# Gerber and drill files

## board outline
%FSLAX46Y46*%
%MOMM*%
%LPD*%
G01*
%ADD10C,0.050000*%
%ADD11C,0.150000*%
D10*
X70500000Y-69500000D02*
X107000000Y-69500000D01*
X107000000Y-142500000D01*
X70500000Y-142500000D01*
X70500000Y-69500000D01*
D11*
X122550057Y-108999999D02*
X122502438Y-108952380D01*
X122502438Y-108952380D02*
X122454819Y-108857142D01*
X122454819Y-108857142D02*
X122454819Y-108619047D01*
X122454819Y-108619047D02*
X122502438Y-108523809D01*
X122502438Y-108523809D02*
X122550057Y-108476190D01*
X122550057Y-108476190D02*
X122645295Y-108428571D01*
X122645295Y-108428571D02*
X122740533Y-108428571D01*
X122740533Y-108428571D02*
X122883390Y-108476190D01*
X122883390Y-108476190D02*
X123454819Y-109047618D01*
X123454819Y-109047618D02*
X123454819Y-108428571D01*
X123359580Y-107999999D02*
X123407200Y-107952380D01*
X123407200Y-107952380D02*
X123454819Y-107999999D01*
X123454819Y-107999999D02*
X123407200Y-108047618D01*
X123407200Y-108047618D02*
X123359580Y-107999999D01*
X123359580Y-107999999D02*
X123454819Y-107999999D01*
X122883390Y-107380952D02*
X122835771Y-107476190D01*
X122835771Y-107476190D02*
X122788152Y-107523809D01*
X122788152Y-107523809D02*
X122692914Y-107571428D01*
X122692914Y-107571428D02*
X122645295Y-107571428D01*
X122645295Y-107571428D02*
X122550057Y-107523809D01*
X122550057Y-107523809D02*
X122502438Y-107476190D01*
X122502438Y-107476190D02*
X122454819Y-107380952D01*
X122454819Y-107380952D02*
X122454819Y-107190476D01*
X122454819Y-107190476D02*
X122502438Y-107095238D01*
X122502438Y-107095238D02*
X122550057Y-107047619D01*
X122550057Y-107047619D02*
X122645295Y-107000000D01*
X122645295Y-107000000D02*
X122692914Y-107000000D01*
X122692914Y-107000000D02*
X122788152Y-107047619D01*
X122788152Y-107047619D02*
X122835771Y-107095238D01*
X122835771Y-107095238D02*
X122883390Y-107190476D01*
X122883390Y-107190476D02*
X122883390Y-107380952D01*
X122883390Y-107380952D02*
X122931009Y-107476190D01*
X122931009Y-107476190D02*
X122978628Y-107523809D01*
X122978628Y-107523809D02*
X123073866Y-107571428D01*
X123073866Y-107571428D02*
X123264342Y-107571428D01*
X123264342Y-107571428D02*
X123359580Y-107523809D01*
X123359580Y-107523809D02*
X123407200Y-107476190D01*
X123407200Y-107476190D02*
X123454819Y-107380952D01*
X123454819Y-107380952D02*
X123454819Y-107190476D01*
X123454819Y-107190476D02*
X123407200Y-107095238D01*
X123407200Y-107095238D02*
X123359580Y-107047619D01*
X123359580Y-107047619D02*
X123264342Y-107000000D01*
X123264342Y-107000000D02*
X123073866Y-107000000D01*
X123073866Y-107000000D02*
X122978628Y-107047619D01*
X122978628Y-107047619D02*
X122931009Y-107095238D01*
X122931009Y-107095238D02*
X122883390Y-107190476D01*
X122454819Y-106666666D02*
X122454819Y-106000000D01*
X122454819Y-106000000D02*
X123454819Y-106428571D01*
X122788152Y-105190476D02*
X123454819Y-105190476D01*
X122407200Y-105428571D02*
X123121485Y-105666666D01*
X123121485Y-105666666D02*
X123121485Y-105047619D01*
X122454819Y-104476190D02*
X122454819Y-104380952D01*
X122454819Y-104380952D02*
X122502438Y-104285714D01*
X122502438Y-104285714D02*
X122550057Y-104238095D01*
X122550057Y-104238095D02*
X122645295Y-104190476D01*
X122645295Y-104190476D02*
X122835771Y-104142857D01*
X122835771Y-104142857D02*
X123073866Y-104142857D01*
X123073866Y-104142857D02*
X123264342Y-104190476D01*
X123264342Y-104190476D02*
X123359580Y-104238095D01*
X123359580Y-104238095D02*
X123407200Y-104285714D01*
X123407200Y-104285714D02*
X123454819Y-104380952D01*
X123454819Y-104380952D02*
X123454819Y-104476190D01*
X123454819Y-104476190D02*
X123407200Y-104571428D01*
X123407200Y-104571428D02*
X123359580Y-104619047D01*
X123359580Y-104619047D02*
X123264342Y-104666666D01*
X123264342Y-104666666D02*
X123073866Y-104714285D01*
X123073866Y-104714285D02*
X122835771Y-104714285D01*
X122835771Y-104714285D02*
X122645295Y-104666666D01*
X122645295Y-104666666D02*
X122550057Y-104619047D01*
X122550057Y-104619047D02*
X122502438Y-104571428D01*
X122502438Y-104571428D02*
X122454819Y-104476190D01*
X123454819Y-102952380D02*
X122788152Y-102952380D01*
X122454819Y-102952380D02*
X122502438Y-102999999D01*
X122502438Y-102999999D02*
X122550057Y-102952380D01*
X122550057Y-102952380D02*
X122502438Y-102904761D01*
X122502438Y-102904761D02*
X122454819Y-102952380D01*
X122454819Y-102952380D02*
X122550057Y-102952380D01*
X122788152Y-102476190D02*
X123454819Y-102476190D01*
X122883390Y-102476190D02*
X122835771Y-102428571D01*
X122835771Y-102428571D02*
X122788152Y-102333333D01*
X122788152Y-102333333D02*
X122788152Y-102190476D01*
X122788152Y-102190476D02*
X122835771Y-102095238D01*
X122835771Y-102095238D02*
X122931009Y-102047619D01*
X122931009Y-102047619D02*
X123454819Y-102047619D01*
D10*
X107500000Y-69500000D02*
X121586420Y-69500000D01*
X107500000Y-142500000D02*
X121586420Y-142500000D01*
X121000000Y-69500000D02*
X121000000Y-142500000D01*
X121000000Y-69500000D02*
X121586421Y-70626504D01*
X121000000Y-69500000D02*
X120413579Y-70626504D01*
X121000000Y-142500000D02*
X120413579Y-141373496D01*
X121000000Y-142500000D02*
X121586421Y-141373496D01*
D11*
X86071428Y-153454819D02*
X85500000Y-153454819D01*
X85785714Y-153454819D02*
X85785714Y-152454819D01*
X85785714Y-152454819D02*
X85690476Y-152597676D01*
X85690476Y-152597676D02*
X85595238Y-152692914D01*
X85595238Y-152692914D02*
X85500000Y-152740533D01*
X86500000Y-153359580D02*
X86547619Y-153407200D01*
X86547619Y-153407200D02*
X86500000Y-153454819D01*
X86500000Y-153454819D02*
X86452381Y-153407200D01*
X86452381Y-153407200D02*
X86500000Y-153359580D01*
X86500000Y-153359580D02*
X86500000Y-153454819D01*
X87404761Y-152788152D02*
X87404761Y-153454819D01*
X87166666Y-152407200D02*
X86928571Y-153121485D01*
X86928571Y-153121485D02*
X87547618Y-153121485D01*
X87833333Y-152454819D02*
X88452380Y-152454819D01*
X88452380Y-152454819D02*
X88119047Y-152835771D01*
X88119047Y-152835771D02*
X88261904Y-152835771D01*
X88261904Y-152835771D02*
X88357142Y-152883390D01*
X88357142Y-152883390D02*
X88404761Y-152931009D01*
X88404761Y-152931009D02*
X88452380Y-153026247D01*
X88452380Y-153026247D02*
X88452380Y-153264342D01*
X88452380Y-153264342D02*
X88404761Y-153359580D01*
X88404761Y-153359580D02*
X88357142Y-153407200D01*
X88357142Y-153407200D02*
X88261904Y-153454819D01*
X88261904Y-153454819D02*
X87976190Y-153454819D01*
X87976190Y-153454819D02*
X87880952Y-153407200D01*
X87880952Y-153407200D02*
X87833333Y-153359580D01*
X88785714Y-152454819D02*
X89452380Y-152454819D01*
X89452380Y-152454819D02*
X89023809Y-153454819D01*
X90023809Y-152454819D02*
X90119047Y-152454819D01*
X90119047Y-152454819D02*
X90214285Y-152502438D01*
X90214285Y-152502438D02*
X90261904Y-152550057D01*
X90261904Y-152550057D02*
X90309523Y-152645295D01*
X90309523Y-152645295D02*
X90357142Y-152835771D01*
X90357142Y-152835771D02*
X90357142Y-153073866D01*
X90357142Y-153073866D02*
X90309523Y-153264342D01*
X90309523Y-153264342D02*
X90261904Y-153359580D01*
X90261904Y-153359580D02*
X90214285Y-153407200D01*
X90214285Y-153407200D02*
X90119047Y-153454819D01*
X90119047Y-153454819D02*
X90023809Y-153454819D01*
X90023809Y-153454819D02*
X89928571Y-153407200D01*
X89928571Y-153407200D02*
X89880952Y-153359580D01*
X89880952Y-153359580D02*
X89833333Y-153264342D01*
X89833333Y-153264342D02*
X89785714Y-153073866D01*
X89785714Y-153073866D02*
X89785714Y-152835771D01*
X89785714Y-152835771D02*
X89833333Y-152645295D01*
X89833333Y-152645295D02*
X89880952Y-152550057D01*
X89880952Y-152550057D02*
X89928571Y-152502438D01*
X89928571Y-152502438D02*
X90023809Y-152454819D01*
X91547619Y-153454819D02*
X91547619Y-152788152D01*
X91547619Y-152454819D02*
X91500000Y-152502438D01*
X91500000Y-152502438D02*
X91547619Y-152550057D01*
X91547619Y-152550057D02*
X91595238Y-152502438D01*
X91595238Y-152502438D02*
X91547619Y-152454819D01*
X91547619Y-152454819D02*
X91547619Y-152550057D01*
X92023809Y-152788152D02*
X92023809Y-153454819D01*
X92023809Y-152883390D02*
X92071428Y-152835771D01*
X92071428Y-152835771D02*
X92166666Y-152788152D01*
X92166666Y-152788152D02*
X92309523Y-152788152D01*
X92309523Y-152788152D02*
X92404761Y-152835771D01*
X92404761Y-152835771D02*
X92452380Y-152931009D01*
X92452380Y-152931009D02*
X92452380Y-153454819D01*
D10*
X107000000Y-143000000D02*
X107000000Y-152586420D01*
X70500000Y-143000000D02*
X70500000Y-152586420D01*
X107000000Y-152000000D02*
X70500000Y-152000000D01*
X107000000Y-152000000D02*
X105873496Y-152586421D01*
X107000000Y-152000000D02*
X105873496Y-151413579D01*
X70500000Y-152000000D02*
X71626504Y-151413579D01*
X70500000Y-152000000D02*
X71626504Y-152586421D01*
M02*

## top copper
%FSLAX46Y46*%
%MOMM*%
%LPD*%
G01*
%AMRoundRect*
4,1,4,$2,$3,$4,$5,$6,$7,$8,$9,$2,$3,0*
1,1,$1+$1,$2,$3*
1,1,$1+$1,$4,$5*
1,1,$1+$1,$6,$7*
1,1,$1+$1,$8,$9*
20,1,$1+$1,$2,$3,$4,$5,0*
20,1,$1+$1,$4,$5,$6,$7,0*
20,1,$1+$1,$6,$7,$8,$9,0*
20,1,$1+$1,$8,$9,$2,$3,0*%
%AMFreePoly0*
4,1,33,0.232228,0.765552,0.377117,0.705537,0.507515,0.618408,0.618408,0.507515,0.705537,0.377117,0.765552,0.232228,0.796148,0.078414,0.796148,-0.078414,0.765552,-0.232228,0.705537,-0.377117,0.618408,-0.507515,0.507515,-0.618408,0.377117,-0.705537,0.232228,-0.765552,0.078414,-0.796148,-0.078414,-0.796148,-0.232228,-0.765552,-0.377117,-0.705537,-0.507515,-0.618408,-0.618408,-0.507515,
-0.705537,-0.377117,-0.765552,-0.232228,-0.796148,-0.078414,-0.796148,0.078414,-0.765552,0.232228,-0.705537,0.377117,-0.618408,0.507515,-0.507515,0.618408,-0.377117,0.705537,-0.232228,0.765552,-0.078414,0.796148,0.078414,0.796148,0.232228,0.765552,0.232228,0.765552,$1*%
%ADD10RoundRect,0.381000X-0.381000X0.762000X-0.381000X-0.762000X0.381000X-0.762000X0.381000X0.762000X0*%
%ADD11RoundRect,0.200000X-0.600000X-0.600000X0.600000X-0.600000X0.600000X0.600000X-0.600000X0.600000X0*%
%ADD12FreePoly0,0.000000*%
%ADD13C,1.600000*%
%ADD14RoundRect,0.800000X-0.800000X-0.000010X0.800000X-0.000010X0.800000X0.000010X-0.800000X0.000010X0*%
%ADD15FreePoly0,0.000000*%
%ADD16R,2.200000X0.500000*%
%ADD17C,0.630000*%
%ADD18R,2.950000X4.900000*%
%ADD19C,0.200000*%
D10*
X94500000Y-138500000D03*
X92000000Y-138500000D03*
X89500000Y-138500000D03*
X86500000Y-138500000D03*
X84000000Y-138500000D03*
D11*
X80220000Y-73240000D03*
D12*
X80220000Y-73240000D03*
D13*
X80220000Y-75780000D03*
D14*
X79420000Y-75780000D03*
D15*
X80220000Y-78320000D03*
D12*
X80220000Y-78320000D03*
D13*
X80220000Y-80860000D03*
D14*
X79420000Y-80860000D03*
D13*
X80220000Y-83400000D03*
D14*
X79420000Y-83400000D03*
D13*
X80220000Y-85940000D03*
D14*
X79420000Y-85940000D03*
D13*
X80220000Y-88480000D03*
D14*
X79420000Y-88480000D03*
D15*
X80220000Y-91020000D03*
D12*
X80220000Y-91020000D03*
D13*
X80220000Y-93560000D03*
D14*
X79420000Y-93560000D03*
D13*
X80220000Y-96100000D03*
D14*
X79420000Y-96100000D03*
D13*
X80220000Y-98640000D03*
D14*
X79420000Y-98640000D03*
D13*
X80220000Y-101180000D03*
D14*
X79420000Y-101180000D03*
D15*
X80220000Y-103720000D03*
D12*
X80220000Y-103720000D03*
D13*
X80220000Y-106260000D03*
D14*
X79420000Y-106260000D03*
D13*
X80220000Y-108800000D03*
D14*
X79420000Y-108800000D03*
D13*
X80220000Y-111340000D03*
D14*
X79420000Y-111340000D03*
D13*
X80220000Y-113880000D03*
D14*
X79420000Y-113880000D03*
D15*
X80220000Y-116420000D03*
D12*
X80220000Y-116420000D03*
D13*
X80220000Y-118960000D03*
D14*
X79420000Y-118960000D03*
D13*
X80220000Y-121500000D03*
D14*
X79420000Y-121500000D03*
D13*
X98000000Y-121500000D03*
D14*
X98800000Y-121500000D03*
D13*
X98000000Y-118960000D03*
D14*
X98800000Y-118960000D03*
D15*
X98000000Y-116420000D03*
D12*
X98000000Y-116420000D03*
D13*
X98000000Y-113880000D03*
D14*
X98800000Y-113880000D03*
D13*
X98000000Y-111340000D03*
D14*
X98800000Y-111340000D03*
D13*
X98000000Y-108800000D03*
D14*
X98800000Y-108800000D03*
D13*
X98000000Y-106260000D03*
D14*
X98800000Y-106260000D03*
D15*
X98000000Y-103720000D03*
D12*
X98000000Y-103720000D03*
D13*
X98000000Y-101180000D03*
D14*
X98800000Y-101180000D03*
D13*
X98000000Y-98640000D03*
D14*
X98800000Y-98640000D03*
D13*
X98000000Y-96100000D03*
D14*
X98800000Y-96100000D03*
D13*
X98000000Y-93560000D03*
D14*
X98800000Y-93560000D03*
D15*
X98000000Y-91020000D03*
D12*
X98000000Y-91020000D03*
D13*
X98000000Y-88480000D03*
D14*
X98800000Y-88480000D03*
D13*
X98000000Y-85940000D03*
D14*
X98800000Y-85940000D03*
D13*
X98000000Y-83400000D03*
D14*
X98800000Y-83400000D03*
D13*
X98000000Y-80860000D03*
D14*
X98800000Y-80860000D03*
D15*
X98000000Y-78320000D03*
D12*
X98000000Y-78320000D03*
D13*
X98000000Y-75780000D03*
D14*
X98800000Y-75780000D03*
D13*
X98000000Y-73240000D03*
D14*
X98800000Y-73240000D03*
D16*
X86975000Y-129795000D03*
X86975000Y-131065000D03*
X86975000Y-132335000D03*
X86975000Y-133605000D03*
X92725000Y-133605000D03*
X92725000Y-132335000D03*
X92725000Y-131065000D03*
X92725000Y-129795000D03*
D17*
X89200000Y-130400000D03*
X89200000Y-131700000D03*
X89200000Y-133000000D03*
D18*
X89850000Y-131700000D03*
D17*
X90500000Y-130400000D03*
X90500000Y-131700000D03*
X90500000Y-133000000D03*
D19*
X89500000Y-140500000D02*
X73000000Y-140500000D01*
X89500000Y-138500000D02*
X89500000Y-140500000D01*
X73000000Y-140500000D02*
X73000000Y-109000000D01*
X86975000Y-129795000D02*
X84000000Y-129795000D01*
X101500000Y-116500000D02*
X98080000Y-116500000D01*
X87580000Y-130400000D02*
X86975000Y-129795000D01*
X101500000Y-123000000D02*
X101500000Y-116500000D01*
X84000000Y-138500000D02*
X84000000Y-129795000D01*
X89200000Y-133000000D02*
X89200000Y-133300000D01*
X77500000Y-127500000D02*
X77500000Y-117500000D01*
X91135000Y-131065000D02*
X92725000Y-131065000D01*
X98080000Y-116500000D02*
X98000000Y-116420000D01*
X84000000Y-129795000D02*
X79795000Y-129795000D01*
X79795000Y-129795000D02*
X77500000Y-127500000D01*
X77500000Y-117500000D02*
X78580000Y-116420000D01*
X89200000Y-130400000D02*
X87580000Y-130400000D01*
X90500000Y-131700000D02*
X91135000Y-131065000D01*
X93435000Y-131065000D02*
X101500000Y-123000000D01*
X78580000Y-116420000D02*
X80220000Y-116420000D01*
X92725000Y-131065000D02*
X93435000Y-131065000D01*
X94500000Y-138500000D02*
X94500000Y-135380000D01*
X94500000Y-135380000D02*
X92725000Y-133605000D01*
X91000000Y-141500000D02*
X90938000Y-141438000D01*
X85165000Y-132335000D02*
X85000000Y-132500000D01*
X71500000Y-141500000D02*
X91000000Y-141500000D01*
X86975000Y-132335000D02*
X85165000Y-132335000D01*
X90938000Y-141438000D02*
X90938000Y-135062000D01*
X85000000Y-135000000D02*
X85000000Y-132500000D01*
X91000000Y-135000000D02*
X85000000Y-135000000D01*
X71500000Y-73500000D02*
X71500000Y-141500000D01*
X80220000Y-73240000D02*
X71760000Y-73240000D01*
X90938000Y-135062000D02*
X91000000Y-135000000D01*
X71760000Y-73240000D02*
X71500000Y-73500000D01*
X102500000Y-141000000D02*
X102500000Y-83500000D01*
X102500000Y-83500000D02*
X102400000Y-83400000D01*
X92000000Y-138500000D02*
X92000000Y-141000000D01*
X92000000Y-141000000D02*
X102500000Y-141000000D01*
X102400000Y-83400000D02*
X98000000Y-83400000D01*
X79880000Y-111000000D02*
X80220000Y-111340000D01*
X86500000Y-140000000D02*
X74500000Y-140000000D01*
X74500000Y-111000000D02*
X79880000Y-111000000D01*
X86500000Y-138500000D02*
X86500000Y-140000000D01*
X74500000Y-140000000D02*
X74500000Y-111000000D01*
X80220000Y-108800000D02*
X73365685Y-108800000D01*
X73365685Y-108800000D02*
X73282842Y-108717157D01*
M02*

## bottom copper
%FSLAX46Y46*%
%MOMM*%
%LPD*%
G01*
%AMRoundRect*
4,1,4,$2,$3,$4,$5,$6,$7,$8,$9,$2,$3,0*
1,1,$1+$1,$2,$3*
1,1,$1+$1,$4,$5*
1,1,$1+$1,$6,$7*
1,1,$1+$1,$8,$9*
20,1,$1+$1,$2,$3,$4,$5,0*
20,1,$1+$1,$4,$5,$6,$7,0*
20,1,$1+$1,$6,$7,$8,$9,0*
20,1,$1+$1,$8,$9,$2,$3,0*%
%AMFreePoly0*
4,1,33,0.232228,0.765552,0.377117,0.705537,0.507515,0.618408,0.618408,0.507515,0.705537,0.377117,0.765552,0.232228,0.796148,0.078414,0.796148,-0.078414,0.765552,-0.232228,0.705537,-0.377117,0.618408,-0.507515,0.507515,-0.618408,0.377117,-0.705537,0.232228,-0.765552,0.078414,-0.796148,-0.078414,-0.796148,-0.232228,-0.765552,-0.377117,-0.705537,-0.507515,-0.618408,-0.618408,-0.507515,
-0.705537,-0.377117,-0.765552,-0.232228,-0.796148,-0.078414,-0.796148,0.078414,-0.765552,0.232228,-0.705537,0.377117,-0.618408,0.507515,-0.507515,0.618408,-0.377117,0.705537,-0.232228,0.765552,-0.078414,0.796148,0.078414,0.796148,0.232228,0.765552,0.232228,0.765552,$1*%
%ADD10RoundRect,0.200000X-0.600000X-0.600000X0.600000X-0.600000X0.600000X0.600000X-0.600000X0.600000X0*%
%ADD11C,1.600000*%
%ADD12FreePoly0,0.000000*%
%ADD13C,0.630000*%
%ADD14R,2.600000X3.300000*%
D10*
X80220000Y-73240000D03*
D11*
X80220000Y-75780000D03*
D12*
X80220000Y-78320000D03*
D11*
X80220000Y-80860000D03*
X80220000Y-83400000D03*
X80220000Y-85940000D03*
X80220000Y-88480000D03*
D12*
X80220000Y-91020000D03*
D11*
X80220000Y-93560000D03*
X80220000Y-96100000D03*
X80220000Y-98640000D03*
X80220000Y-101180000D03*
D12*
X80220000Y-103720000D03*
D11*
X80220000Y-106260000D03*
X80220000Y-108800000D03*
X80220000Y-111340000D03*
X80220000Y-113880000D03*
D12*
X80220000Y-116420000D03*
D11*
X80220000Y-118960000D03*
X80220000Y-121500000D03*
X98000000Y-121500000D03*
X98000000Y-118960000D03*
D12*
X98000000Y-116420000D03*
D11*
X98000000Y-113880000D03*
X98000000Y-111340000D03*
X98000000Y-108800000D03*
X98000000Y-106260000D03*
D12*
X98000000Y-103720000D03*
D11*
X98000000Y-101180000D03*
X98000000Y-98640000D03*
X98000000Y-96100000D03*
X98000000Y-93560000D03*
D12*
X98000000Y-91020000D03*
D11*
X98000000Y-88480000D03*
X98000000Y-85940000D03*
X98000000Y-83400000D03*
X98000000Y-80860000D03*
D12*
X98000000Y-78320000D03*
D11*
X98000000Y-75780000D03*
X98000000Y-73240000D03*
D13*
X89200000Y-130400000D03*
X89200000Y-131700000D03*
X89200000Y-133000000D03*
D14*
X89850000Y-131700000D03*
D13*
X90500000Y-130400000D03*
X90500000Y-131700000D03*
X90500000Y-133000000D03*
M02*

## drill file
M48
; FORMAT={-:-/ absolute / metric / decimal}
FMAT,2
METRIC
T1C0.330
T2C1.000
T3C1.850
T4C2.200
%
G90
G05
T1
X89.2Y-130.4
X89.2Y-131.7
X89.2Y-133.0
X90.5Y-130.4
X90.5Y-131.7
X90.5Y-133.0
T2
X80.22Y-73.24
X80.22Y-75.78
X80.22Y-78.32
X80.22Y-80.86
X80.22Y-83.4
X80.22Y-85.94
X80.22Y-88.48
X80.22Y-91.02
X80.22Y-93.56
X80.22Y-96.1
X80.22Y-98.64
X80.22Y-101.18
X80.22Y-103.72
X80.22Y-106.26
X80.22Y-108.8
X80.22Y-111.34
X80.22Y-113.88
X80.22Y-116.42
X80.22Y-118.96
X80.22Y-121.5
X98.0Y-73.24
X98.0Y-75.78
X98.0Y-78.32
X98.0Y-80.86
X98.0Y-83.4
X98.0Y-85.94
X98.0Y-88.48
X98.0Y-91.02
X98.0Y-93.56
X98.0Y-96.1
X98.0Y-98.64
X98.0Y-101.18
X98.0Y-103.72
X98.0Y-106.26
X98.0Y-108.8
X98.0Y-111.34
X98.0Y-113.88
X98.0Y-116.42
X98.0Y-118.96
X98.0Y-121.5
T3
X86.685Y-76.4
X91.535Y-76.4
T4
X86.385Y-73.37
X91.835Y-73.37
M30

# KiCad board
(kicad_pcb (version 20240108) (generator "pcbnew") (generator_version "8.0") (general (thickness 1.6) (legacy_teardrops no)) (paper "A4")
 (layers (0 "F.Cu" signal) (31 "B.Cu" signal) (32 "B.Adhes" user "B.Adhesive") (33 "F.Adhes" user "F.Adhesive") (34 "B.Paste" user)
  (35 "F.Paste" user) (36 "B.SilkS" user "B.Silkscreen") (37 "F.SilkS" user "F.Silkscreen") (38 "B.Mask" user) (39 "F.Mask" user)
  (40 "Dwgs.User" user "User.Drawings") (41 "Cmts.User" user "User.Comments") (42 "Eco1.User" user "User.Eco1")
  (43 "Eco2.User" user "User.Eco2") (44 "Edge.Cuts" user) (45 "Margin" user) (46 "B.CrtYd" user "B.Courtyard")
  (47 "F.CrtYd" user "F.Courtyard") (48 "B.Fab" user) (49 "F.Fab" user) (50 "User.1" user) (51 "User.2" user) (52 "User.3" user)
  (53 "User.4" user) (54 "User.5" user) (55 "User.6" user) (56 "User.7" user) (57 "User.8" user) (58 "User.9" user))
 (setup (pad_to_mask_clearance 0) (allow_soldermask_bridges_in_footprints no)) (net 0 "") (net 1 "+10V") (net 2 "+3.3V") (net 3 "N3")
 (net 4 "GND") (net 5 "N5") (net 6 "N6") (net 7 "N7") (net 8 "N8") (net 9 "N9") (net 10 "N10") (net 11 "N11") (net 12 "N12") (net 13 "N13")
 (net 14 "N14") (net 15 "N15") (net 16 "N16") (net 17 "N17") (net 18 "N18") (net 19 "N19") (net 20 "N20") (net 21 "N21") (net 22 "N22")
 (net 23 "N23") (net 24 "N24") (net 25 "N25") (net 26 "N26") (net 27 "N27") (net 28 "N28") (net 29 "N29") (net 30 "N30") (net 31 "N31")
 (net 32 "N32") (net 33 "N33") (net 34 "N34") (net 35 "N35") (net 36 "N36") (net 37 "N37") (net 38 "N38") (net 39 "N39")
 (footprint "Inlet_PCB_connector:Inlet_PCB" (layer "F.Cu") (at 89.5 138.5 -90)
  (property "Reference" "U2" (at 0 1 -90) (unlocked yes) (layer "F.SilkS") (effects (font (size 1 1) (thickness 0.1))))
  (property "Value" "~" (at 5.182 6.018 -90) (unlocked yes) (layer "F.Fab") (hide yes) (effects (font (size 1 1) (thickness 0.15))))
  (pad "1" smd roundrect (at 0 -5 270) (size 2.286 1.524) (layers "F.Cu" "F.Paste" "F.Mask") (roundrect_rratio 0.25) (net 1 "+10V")
   (thermal_bridge_angle 45))
  (pad "2" smd roundrect (at 0 -2.5 270) (size 2.286 1.524) (layers "F.Cu" "F.Paste" "F.Mask") (roundrect_rratio 0.25) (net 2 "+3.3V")
   (thermal_bridge_angle 45))
  (pad "3" smd roundrect (at 0 0 270) (size 2.286 1.524) (layers "F.Cu" "F.Paste" "F.Mask") (roundrect_rratio 0.25)
   (thermal_bridge_angle 45))
  (pad "4" smd roundrect (at 0 3 270) (size 2.286 1.524) (layers "F.Cu" "F.Paste" "F.Mask") (roundrect_rratio 0.25) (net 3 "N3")
   (thermal_bridge_angle 45))
  (pad "5" smd roundrect (at 0 5.5 270) (size 2.286 1.524) (layers "F.Cu" "F.Paste" "F.Mask") (roundrect_rratio 0.25) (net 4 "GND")
   (thermal_bridge_angle 45)))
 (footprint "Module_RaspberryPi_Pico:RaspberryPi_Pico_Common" (layer "F.Cu") (at 89.11 97.37)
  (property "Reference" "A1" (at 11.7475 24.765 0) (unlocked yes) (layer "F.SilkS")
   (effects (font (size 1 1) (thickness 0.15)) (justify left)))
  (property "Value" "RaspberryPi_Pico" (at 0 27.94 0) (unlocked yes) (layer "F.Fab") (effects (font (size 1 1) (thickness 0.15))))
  (pad "" np_thru_hole circle (at -2.725 -24) (size 2.2 2.2) (drill 2.2) (layers "*.Mask"))
  (pad "" np_thru_hole circle (at -2.425 -20.97) (size 1.85 1.85) (drill 1.85) (layers "*.Mask"))
  (pad "" np_thru_hole circle (at 2.425 -20.97) (size 1.85 1.85) (drill 1.85) (layers "*.Mask"))
  (pad "" np_thru_hole circle (at 2.725 -24) (size 2.2 2.2) (drill 2.2) (layers "*.Mask"))
  (pad "1" thru_hole roundrect (at -8.89 -24.13) (size 1.6 1.6) (drill 1) (layers "*.Cu" "*.Mask") (remove_unused_layers no)
   (roundrect_rratio 0.125) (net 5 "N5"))
  (pad "1" smd custom (at -8.89 -24.13) (size 1.6 1.6) (layers "F.Cu" "F.Mask") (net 5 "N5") (options (clearance outline) (anchor circle))
   (primitives))
  (pad "2" thru_hole circle (at -8.89 -21.59) (size 1.6 1.6) (drill 1) (layers "*.Cu" "*.Mask") (remove_unused_layers no) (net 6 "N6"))
  (pad "2" smd roundrect (at -8.89 -21.59) (size 3.2 1.6) (drill (offset -0.8 0)) (layers "F.Cu" "F.Mask") (roundrect_rratio 0.5)
   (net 6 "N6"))
  (pad "3" thru_hole custom (at -8.89 -19.05) (size 1.6 1.6) (drill 1) (layers "*.Cu" "*.Mask") (remove_unused_layers no) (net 4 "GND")
   (options (clearance outline) (anchor circle)) (primitives))
  (pad "3" smd custom (at -8.89 -19.05) (size 1.6 1.6) (layers "F.Cu" "F.Mask") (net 4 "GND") (options (clearance outline) (anchor circle))
   (primitives))
  (pad "4" thru_hole circle (at -8.89 -16.51) (size 1.6 1.6) (drill 1) (layers "*.Cu" "*.Mask") (remove_unused_layers no) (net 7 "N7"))
  (pad "4" smd roundrect (at -8.89 -16.51) (size 3.2 1.6) (drill (offset -0.8 0)) (layers "F.Cu" "F.Mask") (roundrect_rratio 0.5)
   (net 7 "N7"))
  (pad "5" thru_hole circle (at -8.89 -13.97) (size 1.6 1.6) (drill 1) (layers "*.Cu" "*.Mask") (remove_unused_layers no) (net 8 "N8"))
  (pad "5" smd roundrect (at -8.89 -13.97) (size 3.2 1.6) (drill (offset -0.8 0)) (layers "F.Cu" "F.Mask") (roundrect_rratio 0.5)
   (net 8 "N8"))
  (pad "6" thru_hole circle (at -8.89 -11.43) (size 1.6 1.6) (drill 1) (layers "*.Cu" "*.Mask") (remove_unused_layers no) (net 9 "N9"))
  (pad "6" smd roundrect (at -8.89 -11.43) (size 3.2 1.6) (drill (offset -0.8 0)) (layers "F.Cu" "F.Mask") (roundrect_rratio 0.5)
   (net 9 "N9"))
  (pad "7" thru_hole circle (at -8.89 -8.89) (size 1.6 1.6) (drill 1) (layers "*.Cu" "*.Mask") (remove_unused_layers no) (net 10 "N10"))
  (pad "7" smd roundrect (at -8.89 -8.89) (size 3.2 1.6) (drill (offset -0.8 0)) (layers "F.Cu" "F.Mask") (roundrect_rratio 0.5)
   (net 10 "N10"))
  (pad "8" thru_hole custom (at -8.89 -6.35) (size 1.6 1.6) (drill 1) (layers "*.Cu" "*.Mask") (remove_unused_layers no) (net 4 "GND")
   (options (clearance outline) (anchor circle)) (primitives))
  (pad "8" smd custom (at -8.89 -6.35) (size 1.6 1.6) (layers "F.Cu" "F.Mask") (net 4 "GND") (options (clearance outline) (anchor circle))
   (primitives))
  (pad "9" thru_hole circle (at -8.89 -3.81) (size 1.6 1.6) (drill 1) (layers "*.Cu" "*.Mask") (remove_unused_layers no) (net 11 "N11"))
  (pad "9" smd roundrect (at -8.89 -3.81) (size 3.2 1.6) (drill (offset -0.8 0)) (layers "F.Cu" "F.Mask") (roundrect_rratio 0.5)
   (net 11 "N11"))
  (pad "10" thru_hole circle (at -8.89 -1.27) (size 1.6 1.6) (drill 1) (layers "*.Cu" "*.Mask") (remove_unused_layers no) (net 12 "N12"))
  (pad "10" smd roundrect (at -8.89 -1.27) (size 3.2 1.6) (drill (offset -0.8 0)) (layers "F.Cu" "F.Mask") (roundrect_rratio 0.5)
   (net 12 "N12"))
  (pad "11" thru_hole circle (at -8.89 1.27) (size 1.6 1.6) (drill 1) (layers "*.Cu" "*.Mask") (remove_unused_layers no) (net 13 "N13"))
  (pad "11" smd roundrect (at -8.89 1.27) (size 3.2 1.6) (drill (offset -0.8 0)) (layers "F.Cu" "F.Mask") (roundrect_rratio 0.5)
   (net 13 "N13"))
  (pad "12" thru_hole circle (at -8.89 3.81) (size 1.6 1.6) (drill 1) (layers "*.Cu" "*.Mask") (remove_unused_layers no) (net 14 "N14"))
  (pad "12" smd roundrect (at -8.89 3.81) (size 3.2 1.6) (drill (offset -0.8 0)) (layers "F.Cu" "F.Mask") (roundrect_rratio 0.5)
   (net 14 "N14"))
  (pad "13" thru_hole custom (at -8.89 6.35) (size 1.6 1.6) (drill 1) (layers "*.Cu" "*.Mask") (remove_unused_layers no) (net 4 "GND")
   (options (clearance outline) (anchor circle)) (primitives))
  (pad "13" smd custom (at -8.89 6.35) (size 1.6 1.6) (layers "F.Cu" "F.Mask") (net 4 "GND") (options (clearance outline) (anchor circle))
   (primitives))
  (pad "14" thru_hole circle (at -8.89 8.89) (size 1.6 1.6) (drill 1) (layers "*.Cu" "*.Mask") (remove_unused_layers no) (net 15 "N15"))
  (pad "14" smd roundrect (at -8.89 8.89) (size 3.2 1.6) (drill (offset -0.8 0)) (layers "F.Cu" "F.Mask") (roundrect_rratio 0.5)
   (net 15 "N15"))
  (pad "15" thru_hole circle (at -8.89 11.43) (size 1.6 1.6) (drill 1) (layers "*.Cu" "*.Mask") (remove_unused_layers no) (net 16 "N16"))
  (pad "15" smd roundrect (at -8.89 11.43) (size 3.2 1.6) (drill (offset -0.8 0)) (layers "F.Cu" "F.Mask") (roundrect_rratio 0.5)
   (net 16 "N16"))
  (pad "16" thru_hole circle (at -8.89 13.97) (size 1.6 1.6) (drill 1) (layers "*.Cu" "*.Mask") (remove_unused_layers no) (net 3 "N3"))
  (pad "16" smd roundrect (at -8.89 13.97) (size 3.2 1.6) (drill (offset -0.8 0)) (layers "F.Cu" "F.Mask") (roundrect_rratio 0.5)
   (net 3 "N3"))
  (pad "17" thru_hole circle (at -8.89 16.51) (size 1.6 1.6) (drill 1) (layers "*.Cu" "*.Mask") (remove_unused_layers no) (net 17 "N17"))
  (pad "17" smd roundrect (at -8.89 16.51) (size 3.2 1.6) (drill (offset -0.8 0)) (layers "F.Cu" "F.Mask") (roundrect_rratio 0.5)
   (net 17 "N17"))
  (pad "18" thru_hole custom (at -8.89 19.05) (size 1.6 1.6) (drill 1) (layers "*.Cu" "*.Mask") (remove_unused_layers no) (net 4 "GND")
   (options (clearance outline) (anchor circle)) (primitives))
  (pad "18" smd custom (at -8.89 19.05) (size 1.6 1.6) (layers "F.Cu" "F.Mask") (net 4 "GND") (options (clearance outline) (anchor circle))
   (primitives))
  (pad "19" thru_hole circle (at -8.89 21.59) (size 1.6 1.6) (drill 1) (layers "*.Cu" "*.Mask") (remove_unused_layers no) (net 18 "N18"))
  (pad "19" smd roundrect (at -8.89 21.59) (size 3.2 1.6) (drill (offset -0.8 0)) (layers "F.Cu" "F.Mask") (roundrect_rratio 0.5)
   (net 18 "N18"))
  (pad "20" thru_hole circle (at -8.89 24.13) (size 1.6 1.6) (drill 1) (layers "*.Cu" "*.Mask") (remove_unused_layers no) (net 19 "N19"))
  (pad "20" smd roundrect (at -8.89 24.13) (size 3.2 1.6) (drill (offset -0.8 0)) (layers "F.Cu" "F.Mask") (roundrect_rratio 0.5)
   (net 19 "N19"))
  (pad "21" thru_hole circle (at 8.89 24.13) (size 1.6 1.6) (drill 1) (layers "*.Cu" "*.Mask") (remove_unused_layers no) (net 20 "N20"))
  (pad "21" smd roundrect (at 8.89 24.13) (size 3.2 1.6) (drill (offset 0.8 0)) (layers "F.Cu" "F.Mask") (roundrect_rratio 0.5)
   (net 20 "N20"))
  (pad "22" thru_hole circle (at 8.89 21.59) (size 1.6 1.6) (drill 1) (layers "*.Cu" "*.Mask") (remove_unused_layers no) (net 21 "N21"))
  (pad "22" smd roundrect (at 8.89 21.59) (size 3.2 1.6) (drill (offset 0.8 0)) (layers "F.Cu" "F.Mask") (roundrect_rratio 0.5)
   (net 21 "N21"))
  (pad "23" thru_hole custom (at 8.89 19.05) (size 1.6 1.6) (drill 1) (layers "*.Cu" "*.Mask") (remove_unused_layers no) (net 4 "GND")
   (options (clearance outline) (anchor circle)) (primitives))
  (pad "23" smd custom (at 8.89 19.05) (size 1.6 1.6) (layers "F.Cu" "F.Mask") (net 4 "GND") (options (clearance outline) (anchor circle))
   (primitives))
  (pad "24" thru_hole circle (at 8.89 16.51) (size 1.6 1.6) (drill 1) (layers "*.Cu" "*.Mask") (remove_unused_layers no) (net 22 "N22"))
  (pad "24" smd roundrect (at 8.89 16.51) (size 3.2 1.6) (drill (offset 0.8 0)) (layers "F.Cu" "F.Mask") (roundrect_rratio 0.5)
   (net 22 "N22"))
  (pad "25" thru_hole circle (at 8.89 13.97) (size 1.6 1.6) (drill 1) (layers "*.Cu" "*.Mask") (remove_unused_layers no) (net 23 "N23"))
  (pad "25" smd roundrect (at 8.89 13.97) (size 3.2 1.6) (drill (offset 0.8 0)) (layers "F.Cu" "F.Mask") (roundrect_rratio 0.5)
   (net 23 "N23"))
  (pad "26" thru_hole circle (at 8.89 11.43) (size 1.6 1.6) (drill 1) (layers "*.Cu" "*.Mask") (remove_unused_layers no) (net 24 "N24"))
  (pad "26" smd roundrect (at 8.89 11.43) (size 3.2 1.6) (drill (offset 0.8 0)) (layers "F.Cu" "F.Mask") (roundrect_rratio 0.5)
   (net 24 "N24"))
  (pad "27" thru_hole circle (at 8.89 8.89) (size 1.6 1.6) (drill 1) (layers "*.Cu" "*.Mask") (remove_unused_layers no) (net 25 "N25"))
  (pad "27" smd roundrect (at 8.89 8.89) (size 3.2 1.6) (drill (offset 0.8 0)) (layers "F.Cu" "F.Mask") (roundrect_rratio 0.5)
   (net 25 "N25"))
  (pad "28" thru_hole custom (at 8.89 6.35) (size 1.6 1.6) (drill 1) (layers "*.Cu" "*.Mask") (remove_unused_layers no) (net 4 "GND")
   (options (clearance outline) (anchor circle)) (primitives))
  (pad "28" smd custom (at 8.89 6.35) (size 1.6 1.6) (layers "F.Cu" "F.Mask") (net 4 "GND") (options (clearance outline) (anchor circle))
   (primitives))
  (pad "29" thru_hole circle (at 8.89 3.81) (size 1.6 1.6) (drill 1) (layers "*.Cu" "*.Mask") (remove_unused_layers no) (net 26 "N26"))
  (pad "29" smd roundrect (at 8.89 3.81) (size 3.2 1.6) (drill (offset 0.8 0)) (layers "F.Cu" "F.Mask") (roundrect_rratio 0.5)
   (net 26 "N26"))
  (pad "30" thru_hole circle (at 8.89 1.27) (size 1.6 1.6) (drill 1) (layers "*.Cu" "*.Mask") (remove_unused_layers no) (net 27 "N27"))
  (pad "30" smd roundrect (at 8.89 1.27) (size 3.2 1.6) (drill (offset 0.8 0)) (layers "F.Cu" "F.Mask") (roundrect_rratio 0.5)
   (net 27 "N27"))
  (pad "31" thru_hole circle (at 8.89 -1.27) (size 1.6 1.6) (drill 1) (layers "*.Cu" "*.Mask") (remove_unused_layers no) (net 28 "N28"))
  (pad "31" smd roundrect (at 8.89 -1.27) (size 3.2 1.6) (drill (offset 0.8 0)) (layers "F.Cu" "F.Mask") (roundrect_rratio 0.5)
   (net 28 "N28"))
  (pad "32" thru_hole circle (at 8.89 -3.81) (size 1.6 1.6) (drill 1) (layers "*.Cu" "*.Mask") (remove_unused_layers no) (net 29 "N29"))
  (pad "32" smd roundrect (at 8.89 -3.81) (size 3.2 1.6) (drill (offset 0.8 0)) (layers "F.Cu" "F.Mask") (roundrect_rratio 0.5)
   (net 29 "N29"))
  (pad "33" thru_hole custom (at 8.89 -6.35) (size 1.6 1.6) (drill 1) (layers "*.Cu" "*.Mask") (remove_unused_layers no) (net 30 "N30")
   (options (clearance outline) (anchor circle)) (primitives))
  (pad "33" smd custom (at 8.89 -6.35) (size 1.6 1.6) (layers "F.Cu" "F.Mask") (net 30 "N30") (options (clearance outline) (anchor circle))
   (primitives))
  (pad "34" thru_hole circle (at 8.89 -8.89) (size 1.6 1.6) (drill 1) (layers "*.Cu" "*.Mask") (remove_unused_layers no) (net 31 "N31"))
  (pad "34" smd roundrect (at 8.89 -8.89) (size 3.2 1.6) (drill (offset 0.8 0)) (layers "F.Cu" "F.Mask") (roundrect_rratio 0.5)
   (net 31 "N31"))
  (pad "35" thru_hole circle (at 8.89 -11.43) (size 1.6 1.6) (drill 1) (layers "*.Cu" "*.Mask") (remove_unused_layers no) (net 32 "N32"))
  (pad "35" smd roundrect (at 8.89 -11.43) (size 3.2 1.6) (drill (offset 0.8 0)) (layers "F.Cu" "F.Mask") (roundrect_rratio 0.5)
   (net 32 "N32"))
  (pad "36" thru_hole circle (at 8.89 -13.97) (size 1.6 1.6) (drill 1) (layers "*.Cu" "*.Mask") (remove_unused_layers no) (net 2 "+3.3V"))
  (pad "36" smd roundrect (at 8.89 -13.97) (size 3.2 1.6) (drill (offset 0.8 0)) (layers "F.Cu" "F.Mask") (roundrect_rratio 0.5)
   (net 2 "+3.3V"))
  (pad "37" thru_hole circle (at 8.89 -16.51) (size 1.6 1.6) (drill 1) (layers "*.Cu" "*.Mask") (remove_unused_layers no) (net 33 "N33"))
  (pad "37" smd roundrect (at 8.89 -16.51) (size 3.2 1.6) (drill (offset 0.8 0)) (layers "F.Cu" "F.Mask") (roundrect_rratio 0.5)
   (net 33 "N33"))
  (pad "38" thru_hole custom (at 8.89 -19.05) (size 1.6 1.6) (drill 1) (layers "*.Cu" "*.Mask") (remove_unused_layers no) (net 4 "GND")
   (options (clearance outline) (anchor circle)) (primitives))
  (pad "38" smd custom (at 8.89 -19.05) (size 1.6 1.6) (layers "F.Cu" "F.Mask") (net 4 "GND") (options (clearance outline) (anchor circle))
   (primitives))
  (pad "39" thru_hole circle (at 8.89 -21.59) (size 1.6 1.6) (drill 1) (layers "*.Cu" "*.Mask") (remove_unused_layers no) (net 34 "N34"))
  (pad "39" smd roundrect (at 8.89 -21.59) (size 3.2 1.6) (drill (offset 0.8 0)) (layers "F.Cu" "F.Mask") (roundrect_rratio 0.5)
   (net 34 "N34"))
  (pad "40" thru_hole circle (at 8.89 -24.13) (size 1.6 1.6) (drill 1) (layers "*.Cu" "*.Mask") (remove_unused_layers no) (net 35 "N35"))
  (pad "40" smd roundrect (at 8.89 -24.13) (size 3.2 1.6) (drill (offset 0.8 0)) (layers "F.Cu" "F.Mask") (roundrect_rratio 0.5)
   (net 35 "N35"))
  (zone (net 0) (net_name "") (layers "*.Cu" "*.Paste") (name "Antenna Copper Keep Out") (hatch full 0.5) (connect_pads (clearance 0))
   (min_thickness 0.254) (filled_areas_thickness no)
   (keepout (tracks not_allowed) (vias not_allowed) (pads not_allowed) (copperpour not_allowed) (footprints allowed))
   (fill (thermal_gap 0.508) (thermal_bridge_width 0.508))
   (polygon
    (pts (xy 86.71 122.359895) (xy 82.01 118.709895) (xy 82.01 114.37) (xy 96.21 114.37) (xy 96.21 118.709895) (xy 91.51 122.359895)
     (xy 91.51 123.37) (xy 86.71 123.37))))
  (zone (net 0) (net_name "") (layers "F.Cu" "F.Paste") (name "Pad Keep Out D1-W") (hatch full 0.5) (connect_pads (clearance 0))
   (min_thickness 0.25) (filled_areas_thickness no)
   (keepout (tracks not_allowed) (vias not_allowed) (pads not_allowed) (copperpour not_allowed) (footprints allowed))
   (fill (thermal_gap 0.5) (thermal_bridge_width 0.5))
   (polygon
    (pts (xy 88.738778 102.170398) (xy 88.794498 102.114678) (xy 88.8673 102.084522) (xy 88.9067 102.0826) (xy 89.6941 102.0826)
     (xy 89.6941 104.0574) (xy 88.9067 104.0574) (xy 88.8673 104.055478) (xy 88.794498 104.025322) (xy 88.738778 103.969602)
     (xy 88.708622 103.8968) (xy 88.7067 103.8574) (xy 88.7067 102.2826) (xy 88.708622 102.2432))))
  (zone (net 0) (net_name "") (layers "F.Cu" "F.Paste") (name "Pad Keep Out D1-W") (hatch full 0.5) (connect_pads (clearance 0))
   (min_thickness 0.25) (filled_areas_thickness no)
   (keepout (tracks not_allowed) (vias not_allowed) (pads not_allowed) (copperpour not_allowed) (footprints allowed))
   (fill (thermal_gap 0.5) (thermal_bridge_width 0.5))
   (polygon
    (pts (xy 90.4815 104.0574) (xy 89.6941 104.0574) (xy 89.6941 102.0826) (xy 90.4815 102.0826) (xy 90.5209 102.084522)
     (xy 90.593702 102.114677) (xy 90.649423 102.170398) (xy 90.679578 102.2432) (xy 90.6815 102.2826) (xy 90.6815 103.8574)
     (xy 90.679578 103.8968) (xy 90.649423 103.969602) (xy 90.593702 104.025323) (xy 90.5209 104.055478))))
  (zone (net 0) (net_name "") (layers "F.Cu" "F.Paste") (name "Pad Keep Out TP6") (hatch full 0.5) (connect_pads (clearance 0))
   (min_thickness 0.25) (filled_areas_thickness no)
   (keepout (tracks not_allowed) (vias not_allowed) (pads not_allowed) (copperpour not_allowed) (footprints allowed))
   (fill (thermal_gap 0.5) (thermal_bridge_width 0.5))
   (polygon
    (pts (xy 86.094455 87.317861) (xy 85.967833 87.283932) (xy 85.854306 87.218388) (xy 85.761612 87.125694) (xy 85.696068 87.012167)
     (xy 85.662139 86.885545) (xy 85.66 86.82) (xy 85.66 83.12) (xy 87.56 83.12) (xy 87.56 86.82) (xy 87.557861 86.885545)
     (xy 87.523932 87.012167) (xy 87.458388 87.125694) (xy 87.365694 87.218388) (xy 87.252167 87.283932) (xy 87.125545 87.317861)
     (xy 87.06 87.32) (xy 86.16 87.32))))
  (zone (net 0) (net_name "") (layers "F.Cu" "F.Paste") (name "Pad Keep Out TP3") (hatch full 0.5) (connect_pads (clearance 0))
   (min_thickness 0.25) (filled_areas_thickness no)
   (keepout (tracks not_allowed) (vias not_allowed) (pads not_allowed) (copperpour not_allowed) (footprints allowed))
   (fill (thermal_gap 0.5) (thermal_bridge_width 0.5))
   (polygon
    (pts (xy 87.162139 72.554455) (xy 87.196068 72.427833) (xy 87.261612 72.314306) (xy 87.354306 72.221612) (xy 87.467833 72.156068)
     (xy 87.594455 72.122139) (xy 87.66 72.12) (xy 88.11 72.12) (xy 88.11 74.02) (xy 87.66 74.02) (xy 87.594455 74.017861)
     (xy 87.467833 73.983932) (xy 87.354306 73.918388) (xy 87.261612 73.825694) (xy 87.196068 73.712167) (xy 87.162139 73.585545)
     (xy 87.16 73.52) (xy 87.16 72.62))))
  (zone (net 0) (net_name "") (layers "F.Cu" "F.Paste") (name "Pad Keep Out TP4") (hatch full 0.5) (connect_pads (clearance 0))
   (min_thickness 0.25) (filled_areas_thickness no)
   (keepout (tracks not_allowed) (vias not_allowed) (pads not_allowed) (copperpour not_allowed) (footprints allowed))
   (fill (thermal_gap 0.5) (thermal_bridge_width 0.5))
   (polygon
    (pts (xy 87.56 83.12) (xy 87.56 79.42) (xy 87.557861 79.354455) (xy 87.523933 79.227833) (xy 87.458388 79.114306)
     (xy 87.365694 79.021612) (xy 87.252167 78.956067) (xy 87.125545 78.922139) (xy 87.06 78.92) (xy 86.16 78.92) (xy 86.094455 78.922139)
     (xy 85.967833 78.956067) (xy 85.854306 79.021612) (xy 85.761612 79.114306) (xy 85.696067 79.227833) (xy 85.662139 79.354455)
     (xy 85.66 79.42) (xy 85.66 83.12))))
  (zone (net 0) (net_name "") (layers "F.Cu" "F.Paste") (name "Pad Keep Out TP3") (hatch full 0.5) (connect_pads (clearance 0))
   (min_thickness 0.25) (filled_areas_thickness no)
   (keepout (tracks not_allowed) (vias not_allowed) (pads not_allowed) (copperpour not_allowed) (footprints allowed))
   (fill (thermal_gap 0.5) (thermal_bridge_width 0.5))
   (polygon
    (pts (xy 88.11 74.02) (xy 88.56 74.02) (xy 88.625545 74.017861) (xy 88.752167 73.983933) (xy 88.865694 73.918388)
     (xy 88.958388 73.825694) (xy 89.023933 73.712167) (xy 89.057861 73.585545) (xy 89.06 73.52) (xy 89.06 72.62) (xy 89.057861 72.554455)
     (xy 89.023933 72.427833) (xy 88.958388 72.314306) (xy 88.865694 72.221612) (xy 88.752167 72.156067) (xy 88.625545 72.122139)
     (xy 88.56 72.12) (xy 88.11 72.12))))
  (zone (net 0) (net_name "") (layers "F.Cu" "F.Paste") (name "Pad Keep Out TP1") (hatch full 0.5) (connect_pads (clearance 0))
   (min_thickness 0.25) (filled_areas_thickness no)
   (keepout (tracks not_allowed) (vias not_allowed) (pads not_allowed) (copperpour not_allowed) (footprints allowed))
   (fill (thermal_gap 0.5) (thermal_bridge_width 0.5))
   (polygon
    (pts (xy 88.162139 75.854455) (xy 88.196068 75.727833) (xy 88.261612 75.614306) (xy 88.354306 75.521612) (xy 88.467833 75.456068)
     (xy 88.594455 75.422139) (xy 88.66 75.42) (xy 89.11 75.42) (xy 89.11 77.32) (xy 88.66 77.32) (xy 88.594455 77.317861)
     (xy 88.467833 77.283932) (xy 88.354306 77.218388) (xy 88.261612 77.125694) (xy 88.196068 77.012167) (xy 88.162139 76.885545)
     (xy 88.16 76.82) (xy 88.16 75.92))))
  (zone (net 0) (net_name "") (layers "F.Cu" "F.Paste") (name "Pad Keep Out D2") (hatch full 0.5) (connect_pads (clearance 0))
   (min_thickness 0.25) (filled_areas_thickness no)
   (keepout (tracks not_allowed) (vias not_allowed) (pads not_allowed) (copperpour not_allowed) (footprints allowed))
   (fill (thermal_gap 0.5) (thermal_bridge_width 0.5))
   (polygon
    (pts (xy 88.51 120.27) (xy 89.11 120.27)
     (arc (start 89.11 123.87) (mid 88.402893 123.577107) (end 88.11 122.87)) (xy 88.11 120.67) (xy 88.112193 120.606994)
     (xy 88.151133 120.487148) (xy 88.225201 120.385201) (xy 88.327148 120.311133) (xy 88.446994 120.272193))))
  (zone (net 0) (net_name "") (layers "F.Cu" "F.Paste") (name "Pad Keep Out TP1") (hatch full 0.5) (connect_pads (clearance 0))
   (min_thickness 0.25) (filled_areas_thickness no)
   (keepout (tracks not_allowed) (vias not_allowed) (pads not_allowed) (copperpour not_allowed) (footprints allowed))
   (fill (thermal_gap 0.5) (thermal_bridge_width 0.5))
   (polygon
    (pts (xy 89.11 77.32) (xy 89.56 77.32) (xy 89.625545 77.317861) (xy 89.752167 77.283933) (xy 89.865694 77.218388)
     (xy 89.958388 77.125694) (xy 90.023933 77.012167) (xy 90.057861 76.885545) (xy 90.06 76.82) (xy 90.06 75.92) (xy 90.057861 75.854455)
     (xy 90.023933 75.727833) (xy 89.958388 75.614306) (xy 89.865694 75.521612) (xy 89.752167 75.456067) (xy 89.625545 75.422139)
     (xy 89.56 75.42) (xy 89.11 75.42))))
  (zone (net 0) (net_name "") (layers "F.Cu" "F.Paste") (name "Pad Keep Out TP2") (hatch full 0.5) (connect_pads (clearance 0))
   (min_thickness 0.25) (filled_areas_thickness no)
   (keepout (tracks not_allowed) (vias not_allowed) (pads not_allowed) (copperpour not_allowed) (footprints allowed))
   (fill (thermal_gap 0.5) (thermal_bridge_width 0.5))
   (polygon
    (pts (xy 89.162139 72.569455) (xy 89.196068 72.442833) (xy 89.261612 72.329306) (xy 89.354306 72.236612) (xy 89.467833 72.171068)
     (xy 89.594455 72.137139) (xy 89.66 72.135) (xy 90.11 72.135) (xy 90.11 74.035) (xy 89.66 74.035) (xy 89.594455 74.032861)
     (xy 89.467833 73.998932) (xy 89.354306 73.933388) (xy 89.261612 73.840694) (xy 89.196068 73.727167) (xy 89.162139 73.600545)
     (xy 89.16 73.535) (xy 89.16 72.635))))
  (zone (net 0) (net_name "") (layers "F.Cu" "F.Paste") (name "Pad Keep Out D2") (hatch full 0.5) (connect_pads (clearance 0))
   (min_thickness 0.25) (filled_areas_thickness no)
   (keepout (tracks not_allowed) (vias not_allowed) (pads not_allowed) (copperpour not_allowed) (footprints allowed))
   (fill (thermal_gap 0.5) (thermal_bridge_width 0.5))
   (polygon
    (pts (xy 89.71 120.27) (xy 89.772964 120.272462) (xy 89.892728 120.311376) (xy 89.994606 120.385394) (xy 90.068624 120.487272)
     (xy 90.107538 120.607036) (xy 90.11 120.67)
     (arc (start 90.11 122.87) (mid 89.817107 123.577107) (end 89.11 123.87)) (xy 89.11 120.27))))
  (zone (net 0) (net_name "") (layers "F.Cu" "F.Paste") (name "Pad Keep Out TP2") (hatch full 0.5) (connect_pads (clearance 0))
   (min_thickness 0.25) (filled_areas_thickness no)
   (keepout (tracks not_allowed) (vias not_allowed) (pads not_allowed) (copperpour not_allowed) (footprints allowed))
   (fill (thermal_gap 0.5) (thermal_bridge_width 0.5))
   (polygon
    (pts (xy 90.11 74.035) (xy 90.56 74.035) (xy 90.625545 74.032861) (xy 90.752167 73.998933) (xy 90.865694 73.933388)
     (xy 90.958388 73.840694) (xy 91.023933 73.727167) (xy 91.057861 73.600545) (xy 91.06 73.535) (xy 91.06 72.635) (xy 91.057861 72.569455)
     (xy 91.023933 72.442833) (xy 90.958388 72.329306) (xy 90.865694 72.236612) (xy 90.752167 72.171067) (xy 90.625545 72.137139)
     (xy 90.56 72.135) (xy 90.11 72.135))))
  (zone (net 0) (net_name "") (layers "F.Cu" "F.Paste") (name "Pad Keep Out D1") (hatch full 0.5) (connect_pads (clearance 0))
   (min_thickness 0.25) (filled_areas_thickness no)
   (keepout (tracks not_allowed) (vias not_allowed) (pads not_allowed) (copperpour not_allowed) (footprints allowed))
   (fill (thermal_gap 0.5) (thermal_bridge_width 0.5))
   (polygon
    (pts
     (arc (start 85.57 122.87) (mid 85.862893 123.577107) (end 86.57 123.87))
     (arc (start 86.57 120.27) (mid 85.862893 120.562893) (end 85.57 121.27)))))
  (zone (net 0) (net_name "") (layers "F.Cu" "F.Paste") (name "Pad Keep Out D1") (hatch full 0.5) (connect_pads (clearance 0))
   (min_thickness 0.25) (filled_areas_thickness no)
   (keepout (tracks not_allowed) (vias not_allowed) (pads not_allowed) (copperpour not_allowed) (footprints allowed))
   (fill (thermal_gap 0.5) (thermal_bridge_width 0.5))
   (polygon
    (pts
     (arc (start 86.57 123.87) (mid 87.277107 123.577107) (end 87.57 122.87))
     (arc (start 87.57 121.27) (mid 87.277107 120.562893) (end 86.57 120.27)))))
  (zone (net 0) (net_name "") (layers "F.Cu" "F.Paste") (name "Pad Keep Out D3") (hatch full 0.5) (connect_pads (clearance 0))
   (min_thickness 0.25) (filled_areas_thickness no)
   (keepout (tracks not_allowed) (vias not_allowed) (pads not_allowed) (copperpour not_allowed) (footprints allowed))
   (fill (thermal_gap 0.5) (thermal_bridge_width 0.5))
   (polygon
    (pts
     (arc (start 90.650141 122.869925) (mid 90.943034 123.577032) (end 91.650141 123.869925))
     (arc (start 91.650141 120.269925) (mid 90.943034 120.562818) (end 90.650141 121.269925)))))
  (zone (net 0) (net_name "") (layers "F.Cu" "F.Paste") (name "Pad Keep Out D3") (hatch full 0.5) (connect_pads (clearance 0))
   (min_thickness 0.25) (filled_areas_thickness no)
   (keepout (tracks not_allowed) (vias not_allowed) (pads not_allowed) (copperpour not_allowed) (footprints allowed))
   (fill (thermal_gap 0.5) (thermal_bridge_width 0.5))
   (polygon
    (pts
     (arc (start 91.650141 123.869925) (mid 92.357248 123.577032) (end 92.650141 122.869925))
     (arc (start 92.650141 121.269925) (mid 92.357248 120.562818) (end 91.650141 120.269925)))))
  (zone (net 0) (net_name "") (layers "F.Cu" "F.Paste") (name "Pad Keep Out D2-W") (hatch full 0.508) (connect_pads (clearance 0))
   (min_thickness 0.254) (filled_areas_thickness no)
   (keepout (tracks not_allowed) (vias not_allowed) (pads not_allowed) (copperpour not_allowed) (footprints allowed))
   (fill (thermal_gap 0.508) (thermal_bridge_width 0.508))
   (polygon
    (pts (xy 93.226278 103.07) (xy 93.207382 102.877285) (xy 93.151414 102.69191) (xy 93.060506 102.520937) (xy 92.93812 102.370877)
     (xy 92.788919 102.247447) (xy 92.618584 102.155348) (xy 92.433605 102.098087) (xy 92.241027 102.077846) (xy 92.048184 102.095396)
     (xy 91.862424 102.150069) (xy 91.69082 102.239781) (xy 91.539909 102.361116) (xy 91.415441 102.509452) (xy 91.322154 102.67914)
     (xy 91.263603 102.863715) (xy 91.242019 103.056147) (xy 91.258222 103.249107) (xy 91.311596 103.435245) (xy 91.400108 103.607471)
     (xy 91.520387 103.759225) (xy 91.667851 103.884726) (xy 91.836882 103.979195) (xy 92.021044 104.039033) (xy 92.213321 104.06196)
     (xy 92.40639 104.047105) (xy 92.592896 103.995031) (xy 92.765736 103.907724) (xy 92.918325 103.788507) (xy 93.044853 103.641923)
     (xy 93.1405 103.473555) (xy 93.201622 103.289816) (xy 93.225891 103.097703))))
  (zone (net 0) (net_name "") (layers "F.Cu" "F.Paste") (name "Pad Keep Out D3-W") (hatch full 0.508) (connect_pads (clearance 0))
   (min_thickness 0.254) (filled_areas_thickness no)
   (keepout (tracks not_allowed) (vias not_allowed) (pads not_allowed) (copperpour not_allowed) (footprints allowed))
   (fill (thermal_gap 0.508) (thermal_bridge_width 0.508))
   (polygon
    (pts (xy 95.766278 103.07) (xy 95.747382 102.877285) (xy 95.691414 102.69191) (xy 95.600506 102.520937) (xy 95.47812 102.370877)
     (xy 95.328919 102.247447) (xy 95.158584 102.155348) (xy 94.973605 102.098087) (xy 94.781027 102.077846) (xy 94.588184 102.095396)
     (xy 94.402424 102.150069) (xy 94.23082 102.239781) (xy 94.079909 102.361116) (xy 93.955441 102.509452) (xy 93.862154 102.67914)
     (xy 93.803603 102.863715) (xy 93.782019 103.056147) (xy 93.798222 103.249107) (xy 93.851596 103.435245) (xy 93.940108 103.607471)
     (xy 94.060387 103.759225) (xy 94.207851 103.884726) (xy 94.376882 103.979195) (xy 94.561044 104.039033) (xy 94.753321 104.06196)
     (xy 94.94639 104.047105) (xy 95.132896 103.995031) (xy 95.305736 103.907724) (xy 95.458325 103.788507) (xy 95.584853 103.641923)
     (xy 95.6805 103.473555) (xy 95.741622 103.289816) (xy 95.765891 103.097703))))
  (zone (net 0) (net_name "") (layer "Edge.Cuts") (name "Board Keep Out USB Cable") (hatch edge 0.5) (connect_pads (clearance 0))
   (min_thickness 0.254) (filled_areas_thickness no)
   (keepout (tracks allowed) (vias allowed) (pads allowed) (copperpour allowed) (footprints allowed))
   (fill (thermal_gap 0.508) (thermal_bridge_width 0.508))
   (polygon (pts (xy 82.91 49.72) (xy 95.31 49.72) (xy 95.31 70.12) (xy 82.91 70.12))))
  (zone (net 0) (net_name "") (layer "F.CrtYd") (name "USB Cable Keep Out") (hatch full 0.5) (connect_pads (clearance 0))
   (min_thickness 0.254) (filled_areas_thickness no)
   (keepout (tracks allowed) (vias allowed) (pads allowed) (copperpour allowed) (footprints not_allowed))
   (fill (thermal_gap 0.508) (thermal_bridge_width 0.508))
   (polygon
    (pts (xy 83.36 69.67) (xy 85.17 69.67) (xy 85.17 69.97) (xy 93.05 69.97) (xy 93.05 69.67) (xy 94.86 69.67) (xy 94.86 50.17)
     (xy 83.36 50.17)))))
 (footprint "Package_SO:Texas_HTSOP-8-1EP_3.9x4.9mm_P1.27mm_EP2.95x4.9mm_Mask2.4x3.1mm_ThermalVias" (layer "F.Cu") (at 89.85 131.7)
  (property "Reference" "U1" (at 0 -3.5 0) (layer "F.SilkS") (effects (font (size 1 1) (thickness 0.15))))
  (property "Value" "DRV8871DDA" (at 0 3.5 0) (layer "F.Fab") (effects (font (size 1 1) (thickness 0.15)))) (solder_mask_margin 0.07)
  (pad "" smd rect (at 0 0) (size 2.4 3.1) (layers "F.Paste")) (pad "" smd rect (at 0 0) (size 2.4 3.1) (layers "F.Mask"))
  (pad "1" smd rect (at -2.875 -1.905) (size 2.2 0.5) (layers "F.Cu" "F.Paste" "F.Mask") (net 4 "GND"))
  (pad "2" smd rect (at -2.875 -0.635) (size 2.2 0.5) (layers "F.Cu" "F.Paste" "F.Mask") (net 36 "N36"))
  (pad "3" smd rect (at -2.875 0.635) (size 2.2 0.5) (layers "F.Cu" "F.Paste" "F.Mask") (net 5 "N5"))
  (pad "4" smd rect (at -2.875 1.905) (size 2.2 0.5) (layers "F.Cu" "F.Paste" "F.Mask") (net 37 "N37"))
  (pad "5" smd rect (at 2.875 1.905) (size 2.2 0.5) (layers "F.Cu" "F.Paste" "F.Mask") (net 1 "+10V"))
  (pad "6" smd rect (at 2.875 0.635) (size 2.2 0.5) (layers "F.Cu" "F.Paste" "F.Mask") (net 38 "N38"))
  (pad "7" smd rect (at 2.875 -0.635) (size 2.2 0.5) (layers "F.Cu" "F.Paste" "F.Mask") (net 4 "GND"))
  (pad "8" smd rect (at 2.875 -1.905) (size 2.2 0.5) (layers "F.Cu" "F.Paste" "F.Mask") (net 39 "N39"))
  (pad "9" thru_hole circle (at -0.65 -1.3) (size 0.63 0.63) (drill 0.33) (layers "*.Cu" "*.Mask") (remove_unused_layers no) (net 4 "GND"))
  (pad "9" thru_hole circle (at -0.65 0) (size 0.63 0.63) (drill 0.33) (layers "*.Cu" "*.Mask") (remove_unused_layers no) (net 4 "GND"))
  (pad "9" thru_hole circle (at -0.65 1.3) (size 0.63 0.63) (drill 0.33) (layers "*.Cu" "*.Mask") (remove_unused_layers no) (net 4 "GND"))
  (pad "9" smd rect (at 0 0) (size 2.6 3.3) (layers "B.Cu") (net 4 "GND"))
  (pad "9" smd rect (at 0 0) (size 2.95 4.9) (layers "F.Cu") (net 4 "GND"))
  (pad "9" thru_hole circle (at 0.65 -1.3) (size 0.63 0.63) (drill 0.33) (layers "*.Cu" "*.Mask") (remove_unused_layers no) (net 4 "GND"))
  (pad "9" thru_hole circle (at 0.65 0) (size 0.63 0.63) (drill 0.33) (layers "*.Cu" "*.Mask") (remove_unused_layers no) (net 4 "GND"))
  (pad "9" thru_hole circle (at 0.65 1.3) (size 0.63 0.63) (drill 0.33) (layers "*.Cu" "*.Mask") (remove_unused_layers no) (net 4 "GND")))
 (gr_rect (start 70.5 69.5) (end 107 142.5) (stroke (width 0.05) (type default)) (fill none) (layer "Edge.Cuts"))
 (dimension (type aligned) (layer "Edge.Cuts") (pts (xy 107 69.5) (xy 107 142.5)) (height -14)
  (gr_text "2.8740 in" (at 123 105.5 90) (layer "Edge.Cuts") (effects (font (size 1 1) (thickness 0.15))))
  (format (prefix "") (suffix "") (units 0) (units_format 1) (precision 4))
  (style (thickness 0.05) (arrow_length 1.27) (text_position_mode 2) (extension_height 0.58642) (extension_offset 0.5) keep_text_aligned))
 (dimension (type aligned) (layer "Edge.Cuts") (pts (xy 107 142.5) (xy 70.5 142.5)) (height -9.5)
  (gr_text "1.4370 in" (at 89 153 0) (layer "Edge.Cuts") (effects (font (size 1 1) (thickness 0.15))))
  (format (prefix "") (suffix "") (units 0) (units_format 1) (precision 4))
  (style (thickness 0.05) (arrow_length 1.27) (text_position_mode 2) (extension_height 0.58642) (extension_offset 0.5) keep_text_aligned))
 (segment (start 89.5 140.5) (end 73 140.5) (width 0.2) (layer "F.Cu") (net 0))
 (segment (start 89.5 138.5) (end 89.5 140.5) (width 0.2) (layer "F.Cu") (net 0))
 (segment (start 73 140.5) (end 73 109) (width 0.2) (layer "F.Cu") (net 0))
 (segment (start 86.975 129.795) (end 84 129.795) (width 0.2) (layer "F.Cu") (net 4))
 (segment (start 101.5 116.5) (end 98.08 116.5) (width 0.2) (layer "F.Cu") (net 4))
 (segment (start 87.58 130.4) (end 86.975 129.795) (width 0.2) (layer "F.Cu") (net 4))
 (segment (start 101.5 123) (end 101.5 116.5) (width 0.2) (layer "F.Cu") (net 4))
 (segment (start 84 138.5) (end 84 129.795) (width 0.2) (layer "F.Cu") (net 4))
 (segment (start 89.2 133) (end 89.2 133.3) (width 0.2) (layer "F.Cu") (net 4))
 (segment (start 77.5 127.5) (end 77.5 117.5) (width 0.2) (layer "F.Cu") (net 4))
 (segment (start 91.135 131.065) (end 92.725 131.065) (width 0.2) (layer "F.Cu") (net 4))
 (segment (start 98.08 116.5) (end 98 116.42) (width 0.2) (layer "F.Cu") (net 4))
 (segment (start 84 129.795) (end 79.795 129.795) (width 0.2) (layer "F.Cu") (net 4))
 (segment (start 79.795 129.795) (end 77.5 127.5) (width 0.2) (layer "F.Cu") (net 4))
 (segment (start 77.5 117.5) (end 78.58 116.42) (width 0.2) (layer "F.Cu") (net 4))
 (segment (start 89.2 130.4) (end 87.58 130.4) (width 0.2) (layer "F.Cu") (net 4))
 (segment (start 90.5 131.7) (end 91.135 131.065) (width 0.2) (layer "F.Cu") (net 4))
 (segment (start 93.435 131.065) (end 101.5 123) (width 0.2) (layer "F.Cu") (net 4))
 (segment (start 78.58 116.42) (end 80.22 116.42) (width 0.2) (layer "F.Cu") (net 4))
 (segment (start 92.725 131.065) (end 93.435 131.065) (width 0.2) (layer "F.Cu") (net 4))
 (segment (start 94.5 138.5) (end 94.5 135.38) (width 0.2) (layer "F.Cu") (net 1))
 (segment (start 94.5 135.38) (end 92.725 133.605) (width 0.2) (layer "F.Cu") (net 1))
 (segment (start 91 141.5) (end 90.938 141.438) (width 0.2) (layer "F.Cu") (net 5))
 (segment (start 85.165 132.335) (end 85 132.5) (width 0.2) (layer "F.Cu") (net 5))
 (segment (start 71.5 141.5) (end 91 141.5) (width 0.2) (layer "F.Cu") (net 5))
 (segment (start 86.975 132.335) (end 85.165 132.335) (width 0.2) (layer "F.Cu") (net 5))
 (segment (start 90.938 141.438) (end 90.938 135.062) (width 0.2) (layer "F.Cu") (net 5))
 (segment (start 85 135) (end 85 132.5) (width 0.2) (layer "F.Cu") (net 5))
 (segment (start 91 135) (end 85 135) (width 0.2) (layer "F.Cu") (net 5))
 (segment (start 71.5 73.5) (end 71.5 141.5) (width 0.2) (layer "F.Cu") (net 5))
 (segment (start 80.22 73.24) (end 71.76 73.24) (width 0.2) (layer "F.Cu") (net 5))
 (segment (start 90.938 135.062) (end 91 135) (width 0.2) (layer "F.Cu") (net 5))
 (segment (start 71.76 73.24) (end 71.5 73.5) (width 0.2) (layer "F.Cu") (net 5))
 (segment (start 102.5 141) (end 102.5 83.5) (width 0.2) (layer "F.Cu") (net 2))
 (segment (start 102.5 83.5) (end 102.4 83.4) (width 0.2) (layer "F.Cu") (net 2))
 (segment (start 92 138.5) (end 92 141) (width 0.2) (layer "F.Cu") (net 2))
 (segment (start 92 141) (end 102.5 141) (width 0.2) (layer "F.Cu") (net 2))
 (segment (start 102.4 83.4) (end 98 83.4) (width 0.2) (layer "F.Cu") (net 2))
 (segment (start 79.88 111) (end 80.22 111.34) (width 0.2) (layer "F.Cu") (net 3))
 (segment (start 86.5 140) (end 74.5 140) (width 0.2) (layer "F.Cu") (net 3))
 (segment (start 74.5 111) (end 79.88 111) (width 0.2) (layer "F.Cu") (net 3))
 (segment (start 86.5 138.5) (end 86.5 140) (width 0.2) (layer "F.Cu") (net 3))
 (segment (start 74.5 140) (end 74.5 111) (width 0.2) (layer "F.Cu") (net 3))
 (segment (start 80.22 108.8) (end 73.365685 108.8) (width 0.2) (layer "F.Cu") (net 16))
 (segment (start 73.365685 108.8) (end 73.282842 108.717157) (width 0.2) (layer "F.Cu") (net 16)))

